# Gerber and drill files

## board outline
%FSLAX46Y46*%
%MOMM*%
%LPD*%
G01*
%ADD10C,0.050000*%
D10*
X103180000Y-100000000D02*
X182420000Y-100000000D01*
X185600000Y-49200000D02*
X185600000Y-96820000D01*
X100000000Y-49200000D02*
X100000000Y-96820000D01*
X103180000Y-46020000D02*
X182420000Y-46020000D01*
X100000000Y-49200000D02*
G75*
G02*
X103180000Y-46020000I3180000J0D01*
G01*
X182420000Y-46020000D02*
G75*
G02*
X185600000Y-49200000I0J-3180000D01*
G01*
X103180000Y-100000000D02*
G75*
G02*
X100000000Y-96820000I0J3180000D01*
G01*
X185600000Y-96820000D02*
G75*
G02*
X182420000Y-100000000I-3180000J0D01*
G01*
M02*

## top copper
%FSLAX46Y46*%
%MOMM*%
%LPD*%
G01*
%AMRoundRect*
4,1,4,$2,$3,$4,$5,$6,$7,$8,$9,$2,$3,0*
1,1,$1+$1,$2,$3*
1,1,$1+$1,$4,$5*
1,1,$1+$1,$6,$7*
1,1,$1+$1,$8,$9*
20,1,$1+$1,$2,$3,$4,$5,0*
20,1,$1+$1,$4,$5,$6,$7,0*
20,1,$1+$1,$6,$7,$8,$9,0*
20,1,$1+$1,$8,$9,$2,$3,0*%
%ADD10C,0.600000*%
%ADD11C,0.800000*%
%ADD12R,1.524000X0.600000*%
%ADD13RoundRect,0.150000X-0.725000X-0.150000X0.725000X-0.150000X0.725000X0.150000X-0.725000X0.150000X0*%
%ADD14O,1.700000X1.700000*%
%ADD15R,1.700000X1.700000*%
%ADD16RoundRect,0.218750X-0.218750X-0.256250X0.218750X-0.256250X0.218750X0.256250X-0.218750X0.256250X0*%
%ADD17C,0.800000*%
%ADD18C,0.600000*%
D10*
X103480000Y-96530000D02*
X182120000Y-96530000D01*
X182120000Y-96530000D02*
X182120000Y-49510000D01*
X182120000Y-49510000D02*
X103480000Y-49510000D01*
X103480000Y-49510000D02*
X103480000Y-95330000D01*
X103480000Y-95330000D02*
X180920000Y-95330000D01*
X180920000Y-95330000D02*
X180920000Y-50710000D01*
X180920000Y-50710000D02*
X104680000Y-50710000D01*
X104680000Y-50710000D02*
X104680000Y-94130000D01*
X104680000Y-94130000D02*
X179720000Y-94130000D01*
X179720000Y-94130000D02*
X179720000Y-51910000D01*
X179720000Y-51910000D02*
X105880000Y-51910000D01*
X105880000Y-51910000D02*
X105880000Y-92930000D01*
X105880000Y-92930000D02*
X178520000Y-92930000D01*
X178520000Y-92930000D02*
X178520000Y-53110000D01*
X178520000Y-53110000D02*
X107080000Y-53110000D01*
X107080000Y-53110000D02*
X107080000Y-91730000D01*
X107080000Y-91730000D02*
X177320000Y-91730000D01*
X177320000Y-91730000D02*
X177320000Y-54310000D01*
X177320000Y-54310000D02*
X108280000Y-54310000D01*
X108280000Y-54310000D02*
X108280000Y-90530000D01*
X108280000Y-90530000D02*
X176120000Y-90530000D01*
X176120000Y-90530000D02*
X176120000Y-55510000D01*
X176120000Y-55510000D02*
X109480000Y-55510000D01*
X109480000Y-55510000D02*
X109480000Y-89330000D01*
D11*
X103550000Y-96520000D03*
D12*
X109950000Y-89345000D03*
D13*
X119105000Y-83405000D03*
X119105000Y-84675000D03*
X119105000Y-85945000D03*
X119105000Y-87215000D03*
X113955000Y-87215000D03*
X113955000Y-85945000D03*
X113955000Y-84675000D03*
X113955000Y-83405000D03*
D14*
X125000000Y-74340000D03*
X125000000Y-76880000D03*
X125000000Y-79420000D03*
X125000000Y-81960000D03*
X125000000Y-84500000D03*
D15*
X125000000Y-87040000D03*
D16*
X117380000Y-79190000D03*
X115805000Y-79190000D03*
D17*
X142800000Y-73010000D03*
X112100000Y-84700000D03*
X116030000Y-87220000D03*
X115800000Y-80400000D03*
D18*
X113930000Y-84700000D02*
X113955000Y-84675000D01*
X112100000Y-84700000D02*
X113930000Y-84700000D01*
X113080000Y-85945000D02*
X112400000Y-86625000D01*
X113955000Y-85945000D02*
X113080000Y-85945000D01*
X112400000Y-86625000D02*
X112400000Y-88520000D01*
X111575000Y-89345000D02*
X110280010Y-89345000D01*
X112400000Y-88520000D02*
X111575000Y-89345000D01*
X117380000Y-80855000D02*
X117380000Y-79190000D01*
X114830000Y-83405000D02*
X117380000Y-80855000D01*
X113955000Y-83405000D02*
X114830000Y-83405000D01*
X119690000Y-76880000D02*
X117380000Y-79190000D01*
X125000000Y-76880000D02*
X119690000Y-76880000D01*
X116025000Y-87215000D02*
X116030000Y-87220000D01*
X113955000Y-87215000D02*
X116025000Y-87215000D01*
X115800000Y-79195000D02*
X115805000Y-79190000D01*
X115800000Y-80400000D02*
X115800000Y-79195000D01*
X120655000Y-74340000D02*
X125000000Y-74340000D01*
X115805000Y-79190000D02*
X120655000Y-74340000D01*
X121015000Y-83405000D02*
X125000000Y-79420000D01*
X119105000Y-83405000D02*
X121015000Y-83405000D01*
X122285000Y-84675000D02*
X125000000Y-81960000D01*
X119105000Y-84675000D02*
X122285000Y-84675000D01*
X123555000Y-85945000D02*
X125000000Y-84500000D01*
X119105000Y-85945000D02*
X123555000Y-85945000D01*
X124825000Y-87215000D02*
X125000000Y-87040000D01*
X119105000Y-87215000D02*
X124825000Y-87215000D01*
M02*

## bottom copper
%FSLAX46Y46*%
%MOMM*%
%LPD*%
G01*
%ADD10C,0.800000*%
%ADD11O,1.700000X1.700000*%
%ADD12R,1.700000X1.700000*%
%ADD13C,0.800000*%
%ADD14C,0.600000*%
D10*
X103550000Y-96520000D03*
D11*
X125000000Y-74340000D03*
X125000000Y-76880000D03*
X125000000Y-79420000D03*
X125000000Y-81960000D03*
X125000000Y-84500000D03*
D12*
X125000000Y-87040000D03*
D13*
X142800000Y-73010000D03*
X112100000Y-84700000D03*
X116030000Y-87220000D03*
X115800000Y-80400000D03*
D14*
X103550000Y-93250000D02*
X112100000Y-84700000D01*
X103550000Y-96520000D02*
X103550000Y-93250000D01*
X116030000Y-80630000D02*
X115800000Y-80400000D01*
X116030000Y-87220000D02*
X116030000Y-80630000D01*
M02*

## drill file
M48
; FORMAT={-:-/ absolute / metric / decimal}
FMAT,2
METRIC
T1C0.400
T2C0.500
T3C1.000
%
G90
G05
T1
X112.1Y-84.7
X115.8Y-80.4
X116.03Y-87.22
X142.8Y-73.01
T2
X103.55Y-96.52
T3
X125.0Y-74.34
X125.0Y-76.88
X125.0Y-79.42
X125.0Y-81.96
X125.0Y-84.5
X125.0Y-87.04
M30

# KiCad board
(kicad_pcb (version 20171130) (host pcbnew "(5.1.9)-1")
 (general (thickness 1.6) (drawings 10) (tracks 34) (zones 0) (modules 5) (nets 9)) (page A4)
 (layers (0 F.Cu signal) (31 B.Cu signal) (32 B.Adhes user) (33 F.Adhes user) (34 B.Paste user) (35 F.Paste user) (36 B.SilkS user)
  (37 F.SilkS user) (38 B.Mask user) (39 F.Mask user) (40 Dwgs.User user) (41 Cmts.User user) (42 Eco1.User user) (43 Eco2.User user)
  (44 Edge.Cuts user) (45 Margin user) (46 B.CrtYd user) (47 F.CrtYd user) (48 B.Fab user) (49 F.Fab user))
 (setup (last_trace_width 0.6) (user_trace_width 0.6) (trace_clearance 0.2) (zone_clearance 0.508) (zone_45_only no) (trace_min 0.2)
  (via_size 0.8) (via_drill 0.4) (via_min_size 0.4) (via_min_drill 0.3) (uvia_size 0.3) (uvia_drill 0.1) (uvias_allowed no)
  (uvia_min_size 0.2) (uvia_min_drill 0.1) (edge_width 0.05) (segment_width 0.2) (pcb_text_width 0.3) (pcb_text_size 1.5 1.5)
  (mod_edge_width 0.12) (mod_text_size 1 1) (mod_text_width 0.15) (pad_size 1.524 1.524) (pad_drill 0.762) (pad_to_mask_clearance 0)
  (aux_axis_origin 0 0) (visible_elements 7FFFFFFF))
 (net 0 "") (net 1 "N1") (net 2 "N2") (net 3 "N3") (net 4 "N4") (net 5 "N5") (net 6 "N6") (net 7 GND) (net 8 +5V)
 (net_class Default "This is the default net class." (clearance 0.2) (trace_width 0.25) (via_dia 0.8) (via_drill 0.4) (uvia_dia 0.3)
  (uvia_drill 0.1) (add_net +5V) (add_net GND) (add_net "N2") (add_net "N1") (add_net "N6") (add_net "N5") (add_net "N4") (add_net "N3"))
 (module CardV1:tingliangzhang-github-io (layer F.Cu) (at 163.77 73.62)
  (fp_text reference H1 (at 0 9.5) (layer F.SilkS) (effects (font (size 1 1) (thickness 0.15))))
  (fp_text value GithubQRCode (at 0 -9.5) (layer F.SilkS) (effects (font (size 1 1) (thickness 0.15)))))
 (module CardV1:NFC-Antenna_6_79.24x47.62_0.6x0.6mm (layer F.Cu) (at 142.8 73.02)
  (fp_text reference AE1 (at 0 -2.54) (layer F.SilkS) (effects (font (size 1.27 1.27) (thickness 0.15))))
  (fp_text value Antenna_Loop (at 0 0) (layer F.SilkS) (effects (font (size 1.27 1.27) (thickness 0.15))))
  (fp_line (start -39.32 23.51) (end 39.32 23.51) (layer F.Cu) (width 0.6))
  (fp_line (start 39.32 23.51) (end 39.32 -23.51) (layer F.Cu) (width 0.6))
  (fp_line (start 39.32 -23.51) (end -39.32 -23.51) (layer F.Cu) (width 0.6))
  (fp_line (start -39.32 -23.51) (end -39.32 22.31) (layer F.Cu) (width 0.6))
  (fp_line (start -39.32 22.31) (end 38.12 22.31) (layer F.Cu) (width 0.6))
  (fp_line (start 38.12 22.31) (end 38.12 -22.31) (layer F.Cu) (width 0.6))
  (fp_line (start 38.12 -22.31) (end -38.12 -22.31) (layer F.Cu) (width 0.6))
  (fp_line (start -38.12 -22.31) (end -38.12 21.11) (layer F.Cu) (width 0.6))
  (fp_line (start -38.12 21.11) (end 36.92 21.11) (layer F.Cu) (width 0.6))
  (fp_line (start 36.92 21.11) (end 36.92 -21.11) (layer F.Cu) (width 0.6))
  (fp_line (start 36.92 -21.11) (end -36.92 -21.11) (layer F.Cu) (width 0.6))
  (fp_line (start -36.92 -21.11) (end -36.92 19.91) (layer F.Cu) (width 0.6))
  (fp_line (start -36.92 19.91) (end 35.72 19.91) (layer F.Cu) (width 0.6))
  (fp_line (start 35.72 19.91) (end 35.72 -19.91) (layer F.Cu) (width 0.6))
  (fp_line (start 35.72 -19.91) (end -35.72 -19.91) (layer F.Cu) (width 0.6))
  (fp_line (start -35.72 -19.91) (end -35.72 18.71) (layer F.Cu) (width 0.6))
  (fp_line (start -35.72 18.71) (end 34.52 18.71) (layer F.Cu) (width 0.6))
  (fp_line (start 34.52 18.71) (end 34.52 -18.71) (layer F.Cu) (width 0.6))
  (fp_line (start 34.52 -18.71) (end -34.52 -18.71) (layer F.Cu) (width 0.6))
  (fp_line (start -34.52 -18.71) (end -34.52 17.51) (layer F.Cu) (width 0.6))
  (fp_line (start -34.52 17.51) (end 33.32 17.51) (layer F.Cu) (width 0.6))
  (fp_line (start 33.32 17.51) (end 33.32 -17.51) (layer F.Cu) (width 0.6))
  (fp_line (start 33.32 -17.51) (end -33.32 -17.51) (layer F.Cu) (width 0.6))
  (fp_line (start -33.32 -17.51) (end -33.32 16.31) (layer F.Cu) (width 0.6))
  (pad 2 thru_hole circle (at -39.25 23.5) (size 0.8 0.8) (drill 0.5) (layers *.Cu) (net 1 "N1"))
  (pad 1 smd rect (at -32.85 16.325) (size 1.524 0.6) (layers F.Cu) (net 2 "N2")))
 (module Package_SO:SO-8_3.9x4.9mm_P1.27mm (layer F.Cu) (at 116.53 85.31)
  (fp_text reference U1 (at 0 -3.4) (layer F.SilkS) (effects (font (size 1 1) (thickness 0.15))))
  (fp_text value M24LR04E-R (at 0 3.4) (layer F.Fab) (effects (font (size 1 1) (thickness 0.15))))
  (pad 8 smd roundrect (at 2.575 -1.905) (size 1.75 0.6) (layers F.Cu F.Paste F.Mask) (roundrect_rratio 0.25) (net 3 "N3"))
  (pad 7 smd roundrect (at 2.575 -0.635) (size 1.75 0.6) (layers F.Cu F.Paste F.Mask) (roundrect_rratio 0.25) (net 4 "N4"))
  (pad 6 smd roundrect (at 2.575 0.635) (size 1.75 0.6) (layers F.Cu F.Paste F.Mask) (roundrect_rratio 0.25) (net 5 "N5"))
  (pad 5 smd roundrect (at 2.575 1.905) (size 1.75 0.6) (layers F.Cu F.Paste F.Mask) (roundrect_rratio 0.25) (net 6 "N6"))
  (pad 4 smd roundrect (at -2.575 1.905) (size 1.75 0.6) (layers F.Cu F.Paste F.Mask) (roundrect_rratio 0.25) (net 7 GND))
  (pad 3 smd roundrect (at -2.575 0.635) (size 1.75 0.6) (layers F.Cu F.Paste F.Mask) (roundrect_rratio 0.25) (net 2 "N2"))
  (pad 2 smd roundrect (at -2.575 -0.635) (size 1.75 0.6) (layers F.Cu F.Paste F.Mask) (roundrect_rratio 0.25) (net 1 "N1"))
  (pad 1 smd roundrect (at -2.575 -1.905) (size 1.75 0.6) (layers F.Cu F.Paste F.Mask) (roundrect_rratio 0.25) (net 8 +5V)))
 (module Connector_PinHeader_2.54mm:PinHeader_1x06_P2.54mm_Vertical (layer F.Cu) (at 125 87.04 180)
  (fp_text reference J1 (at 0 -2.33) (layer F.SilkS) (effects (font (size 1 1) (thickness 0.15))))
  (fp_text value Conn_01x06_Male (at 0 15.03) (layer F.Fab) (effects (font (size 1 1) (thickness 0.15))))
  (pad 6 thru_hole oval (at 0 12.7 180) (size 1.7 1.7) (drill 1) (layers *.Cu *.Mask) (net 7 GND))
  (pad 5 thru_hole oval (at 0 10.16 180) (size 1.7 1.7) (drill 1) (layers *.Cu *.Mask) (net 8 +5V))
  (pad 4 thru_hole oval (at 0 7.62 180) (size 1.7 1.7) (drill 1) (layers *.Cu *.Mask) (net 3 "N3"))
  (pad 3 thru_hole oval (at 0 5.08 180) (size 1.7 1.7) (drill 1) (layers *.Cu *.Mask) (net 4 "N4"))
  (pad 2 thru_hole oval (at 0 2.54 180) (size 1.7 1.7) (drill 1) (layers *.Cu *.Mask) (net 5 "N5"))
  (pad 1 thru_hole rect (at 0 0 180) (size 1.7 1.7) (drill 1) (layers *.Cu *.Mask) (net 6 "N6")))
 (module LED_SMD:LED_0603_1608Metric (layer F.Cu) (at 116.5925 79.19)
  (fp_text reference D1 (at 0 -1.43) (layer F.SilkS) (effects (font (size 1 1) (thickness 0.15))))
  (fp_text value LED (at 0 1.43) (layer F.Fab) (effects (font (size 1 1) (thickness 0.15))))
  (pad 2 smd roundrect (at 0.7875 0) (size 0.875 0.95) (layers F.Cu F.Paste F.Mask) (roundrect_rratio 0.25) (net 8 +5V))
  (pad 1 smd roundrect (at -0.7875 0) (size 0.875 0.95) (layers F.Cu F.Paste F.Mask) (roundrect_rratio 0.25) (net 7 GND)))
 (gr_line (start 103.18 100) (end 182.42 100) (layer Edge.Cuts) (width 0.05))
 (gr_line (start 185.6 49.2) (end 185.6 96.82) (layer Edge.Cuts) (width 0.05))
 (gr_line (start 100 49.2) (end 100 96.82) (layer Edge.Cuts) (width 0.05))
 (gr_line (start 103.18 46.02) (end 182.42 46.02) (layer Edge.Cuts) (width 0.05))
 (gr_arc (start 103.18 49.2) (end 103.18 46.02) (angle -90) (layer Edge.Cuts) (width 0.05))
 (gr_arc (start 182.42 49.2) (end 185.6 49.2) (angle -90) (layer Edge.Cuts) (width 0.05))
 (gr_arc (start 103.18 96.82) (end 100 96.82) (angle -90) (layer Edge.Cuts) (width 0.05))
 (gr_arc (start 182.42 96.82) (end 182.42 100) (angle -90) (layer Edge.Cuts) (width 0.05))
 (via (at 142.8 73.01) (size 0.8) (drill 0.4) (layers F.Cu B.Cu) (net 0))
 (via (at 112.1 84.7) (size 0.8) (drill 0.4) (layers F.Cu B.Cu) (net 1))
 (segment (start 103.55 93.25) (end 112.1 84.7) (width 0.6) (layer B.Cu) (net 1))
 (segment (start 103.55 96.52) (end 103.55 93.25) (width 0.6) (layer B.Cu) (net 1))
 (segment (start 113.93 84.7) (end 113.955 84.675) (width 0.6) (layer F.Cu) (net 1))
 (segment (start 112.1 84.7) (end 113.93 84.7) (width 0.6) (layer F.Cu) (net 1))
 (segment (start 113.08 85.945) (end 112.4 86.625) (width 0.6) (layer F.Cu) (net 2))
 (segment (start 113.955 85.945) (end 113.08 85.945) (width 0.6) (layer F.Cu) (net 2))
 (segment (start 112.4 86.625) (end 112.4 88.52) (width 0.6) (layer F.Cu) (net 2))
 (segment (start 111.575 89.345) (end 110.28001 89.345) (width 0.6) (layer F.Cu) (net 2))
 (segment (start 112.4 88.52) (end 111.575 89.345) (width 0.6) (layer F.Cu) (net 2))
 (segment (start 117.38 80.855) (end 117.38 79.19) (width 0.6) (layer F.Cu) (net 8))
 (segment (start 114.83 83.405) (end 117.38 80.855) (width 0.6) (layer F.Cu) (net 8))
 (segment (start 113.955 83.405) (end 114.83 83.405) (width 0.6) (layer F.Cu) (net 8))
 (segment (start 119.69 76.88) (end 117.38 79.19) (width 0.6) (layer F.Cu) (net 8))
 (segment (start 125 76.88) (end 119.69 76.88) (width 0.6) (layer F.Cu) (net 8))
 (via (at 116.03 87.22) (size 0.8) (drill 0.4) (layers F.Cu B.Cu) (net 7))
 (segment (start 116.025 87.215) (end 116.03 87.22) (width 0.6) (layer F.Cu) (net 7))
 (segment (start 113.955 87.215) (end 116.025 87.215) (width 0.6) (layer F.Cu) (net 7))
 (via (at 115.8 80.4) (size 0.8) (drill 0.4) (layers F.Cu B.Cu) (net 7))
 (segment (start 116.03 80.63) (end 115.8 80.4) (width 0.6) (layer B.Cu) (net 7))
 (segment (start 116.03 87.22) (end 116.03 80.63) (width 0.6) (layer B.Cu) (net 7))
 (segment (start 115.8 79.195) (end 115.805 79.19) (width 0.6) (layer F.Cu) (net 7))
 (segment (start 115.8 80.4) (end 115.8 79.195) (width 0.6) (layer F.Cu) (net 7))
 (segment (start 120.655 74.34) (end 125 74.34) (width 0.6) (layer F.Cu) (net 7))
 (segment (start 115.805 79.19) (end 120.655 74.34) (width 0.6) (layer F.Cu) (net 7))
 (segment (start 121.015 83.405) (end 125 79.42) (width 0.6) (layer F.Cu) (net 3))
 (segment (start 119.105 83.405) (end 121.015 83.405) (width 0.6) (layer F.Cu) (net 3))
 (segment (start 122.285 84.675) (end 125 81.96) (width 0.6) (layer F.Cu) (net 4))
 (segment (start 119.105 84.675) (end 122.285 84.675) (width 0.6) (layer F.Cu) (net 4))
 (segment (start 123.555 85.945) (end 125 84.5) (width 0.6) (layer F.Cu) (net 5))
 (segment (start 119.105 85.945) (end 123.555 85.945) (width 0.6) (layer F.Cu) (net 5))
 (segment (start 124.825 87.215) (end 125 87.04) (width 0.6) (layer F.Cu) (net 6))
 (segment (start 119.105 87.215) (end 124.825 87.215) (width 0.6) (layer F.Cu) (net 6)))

